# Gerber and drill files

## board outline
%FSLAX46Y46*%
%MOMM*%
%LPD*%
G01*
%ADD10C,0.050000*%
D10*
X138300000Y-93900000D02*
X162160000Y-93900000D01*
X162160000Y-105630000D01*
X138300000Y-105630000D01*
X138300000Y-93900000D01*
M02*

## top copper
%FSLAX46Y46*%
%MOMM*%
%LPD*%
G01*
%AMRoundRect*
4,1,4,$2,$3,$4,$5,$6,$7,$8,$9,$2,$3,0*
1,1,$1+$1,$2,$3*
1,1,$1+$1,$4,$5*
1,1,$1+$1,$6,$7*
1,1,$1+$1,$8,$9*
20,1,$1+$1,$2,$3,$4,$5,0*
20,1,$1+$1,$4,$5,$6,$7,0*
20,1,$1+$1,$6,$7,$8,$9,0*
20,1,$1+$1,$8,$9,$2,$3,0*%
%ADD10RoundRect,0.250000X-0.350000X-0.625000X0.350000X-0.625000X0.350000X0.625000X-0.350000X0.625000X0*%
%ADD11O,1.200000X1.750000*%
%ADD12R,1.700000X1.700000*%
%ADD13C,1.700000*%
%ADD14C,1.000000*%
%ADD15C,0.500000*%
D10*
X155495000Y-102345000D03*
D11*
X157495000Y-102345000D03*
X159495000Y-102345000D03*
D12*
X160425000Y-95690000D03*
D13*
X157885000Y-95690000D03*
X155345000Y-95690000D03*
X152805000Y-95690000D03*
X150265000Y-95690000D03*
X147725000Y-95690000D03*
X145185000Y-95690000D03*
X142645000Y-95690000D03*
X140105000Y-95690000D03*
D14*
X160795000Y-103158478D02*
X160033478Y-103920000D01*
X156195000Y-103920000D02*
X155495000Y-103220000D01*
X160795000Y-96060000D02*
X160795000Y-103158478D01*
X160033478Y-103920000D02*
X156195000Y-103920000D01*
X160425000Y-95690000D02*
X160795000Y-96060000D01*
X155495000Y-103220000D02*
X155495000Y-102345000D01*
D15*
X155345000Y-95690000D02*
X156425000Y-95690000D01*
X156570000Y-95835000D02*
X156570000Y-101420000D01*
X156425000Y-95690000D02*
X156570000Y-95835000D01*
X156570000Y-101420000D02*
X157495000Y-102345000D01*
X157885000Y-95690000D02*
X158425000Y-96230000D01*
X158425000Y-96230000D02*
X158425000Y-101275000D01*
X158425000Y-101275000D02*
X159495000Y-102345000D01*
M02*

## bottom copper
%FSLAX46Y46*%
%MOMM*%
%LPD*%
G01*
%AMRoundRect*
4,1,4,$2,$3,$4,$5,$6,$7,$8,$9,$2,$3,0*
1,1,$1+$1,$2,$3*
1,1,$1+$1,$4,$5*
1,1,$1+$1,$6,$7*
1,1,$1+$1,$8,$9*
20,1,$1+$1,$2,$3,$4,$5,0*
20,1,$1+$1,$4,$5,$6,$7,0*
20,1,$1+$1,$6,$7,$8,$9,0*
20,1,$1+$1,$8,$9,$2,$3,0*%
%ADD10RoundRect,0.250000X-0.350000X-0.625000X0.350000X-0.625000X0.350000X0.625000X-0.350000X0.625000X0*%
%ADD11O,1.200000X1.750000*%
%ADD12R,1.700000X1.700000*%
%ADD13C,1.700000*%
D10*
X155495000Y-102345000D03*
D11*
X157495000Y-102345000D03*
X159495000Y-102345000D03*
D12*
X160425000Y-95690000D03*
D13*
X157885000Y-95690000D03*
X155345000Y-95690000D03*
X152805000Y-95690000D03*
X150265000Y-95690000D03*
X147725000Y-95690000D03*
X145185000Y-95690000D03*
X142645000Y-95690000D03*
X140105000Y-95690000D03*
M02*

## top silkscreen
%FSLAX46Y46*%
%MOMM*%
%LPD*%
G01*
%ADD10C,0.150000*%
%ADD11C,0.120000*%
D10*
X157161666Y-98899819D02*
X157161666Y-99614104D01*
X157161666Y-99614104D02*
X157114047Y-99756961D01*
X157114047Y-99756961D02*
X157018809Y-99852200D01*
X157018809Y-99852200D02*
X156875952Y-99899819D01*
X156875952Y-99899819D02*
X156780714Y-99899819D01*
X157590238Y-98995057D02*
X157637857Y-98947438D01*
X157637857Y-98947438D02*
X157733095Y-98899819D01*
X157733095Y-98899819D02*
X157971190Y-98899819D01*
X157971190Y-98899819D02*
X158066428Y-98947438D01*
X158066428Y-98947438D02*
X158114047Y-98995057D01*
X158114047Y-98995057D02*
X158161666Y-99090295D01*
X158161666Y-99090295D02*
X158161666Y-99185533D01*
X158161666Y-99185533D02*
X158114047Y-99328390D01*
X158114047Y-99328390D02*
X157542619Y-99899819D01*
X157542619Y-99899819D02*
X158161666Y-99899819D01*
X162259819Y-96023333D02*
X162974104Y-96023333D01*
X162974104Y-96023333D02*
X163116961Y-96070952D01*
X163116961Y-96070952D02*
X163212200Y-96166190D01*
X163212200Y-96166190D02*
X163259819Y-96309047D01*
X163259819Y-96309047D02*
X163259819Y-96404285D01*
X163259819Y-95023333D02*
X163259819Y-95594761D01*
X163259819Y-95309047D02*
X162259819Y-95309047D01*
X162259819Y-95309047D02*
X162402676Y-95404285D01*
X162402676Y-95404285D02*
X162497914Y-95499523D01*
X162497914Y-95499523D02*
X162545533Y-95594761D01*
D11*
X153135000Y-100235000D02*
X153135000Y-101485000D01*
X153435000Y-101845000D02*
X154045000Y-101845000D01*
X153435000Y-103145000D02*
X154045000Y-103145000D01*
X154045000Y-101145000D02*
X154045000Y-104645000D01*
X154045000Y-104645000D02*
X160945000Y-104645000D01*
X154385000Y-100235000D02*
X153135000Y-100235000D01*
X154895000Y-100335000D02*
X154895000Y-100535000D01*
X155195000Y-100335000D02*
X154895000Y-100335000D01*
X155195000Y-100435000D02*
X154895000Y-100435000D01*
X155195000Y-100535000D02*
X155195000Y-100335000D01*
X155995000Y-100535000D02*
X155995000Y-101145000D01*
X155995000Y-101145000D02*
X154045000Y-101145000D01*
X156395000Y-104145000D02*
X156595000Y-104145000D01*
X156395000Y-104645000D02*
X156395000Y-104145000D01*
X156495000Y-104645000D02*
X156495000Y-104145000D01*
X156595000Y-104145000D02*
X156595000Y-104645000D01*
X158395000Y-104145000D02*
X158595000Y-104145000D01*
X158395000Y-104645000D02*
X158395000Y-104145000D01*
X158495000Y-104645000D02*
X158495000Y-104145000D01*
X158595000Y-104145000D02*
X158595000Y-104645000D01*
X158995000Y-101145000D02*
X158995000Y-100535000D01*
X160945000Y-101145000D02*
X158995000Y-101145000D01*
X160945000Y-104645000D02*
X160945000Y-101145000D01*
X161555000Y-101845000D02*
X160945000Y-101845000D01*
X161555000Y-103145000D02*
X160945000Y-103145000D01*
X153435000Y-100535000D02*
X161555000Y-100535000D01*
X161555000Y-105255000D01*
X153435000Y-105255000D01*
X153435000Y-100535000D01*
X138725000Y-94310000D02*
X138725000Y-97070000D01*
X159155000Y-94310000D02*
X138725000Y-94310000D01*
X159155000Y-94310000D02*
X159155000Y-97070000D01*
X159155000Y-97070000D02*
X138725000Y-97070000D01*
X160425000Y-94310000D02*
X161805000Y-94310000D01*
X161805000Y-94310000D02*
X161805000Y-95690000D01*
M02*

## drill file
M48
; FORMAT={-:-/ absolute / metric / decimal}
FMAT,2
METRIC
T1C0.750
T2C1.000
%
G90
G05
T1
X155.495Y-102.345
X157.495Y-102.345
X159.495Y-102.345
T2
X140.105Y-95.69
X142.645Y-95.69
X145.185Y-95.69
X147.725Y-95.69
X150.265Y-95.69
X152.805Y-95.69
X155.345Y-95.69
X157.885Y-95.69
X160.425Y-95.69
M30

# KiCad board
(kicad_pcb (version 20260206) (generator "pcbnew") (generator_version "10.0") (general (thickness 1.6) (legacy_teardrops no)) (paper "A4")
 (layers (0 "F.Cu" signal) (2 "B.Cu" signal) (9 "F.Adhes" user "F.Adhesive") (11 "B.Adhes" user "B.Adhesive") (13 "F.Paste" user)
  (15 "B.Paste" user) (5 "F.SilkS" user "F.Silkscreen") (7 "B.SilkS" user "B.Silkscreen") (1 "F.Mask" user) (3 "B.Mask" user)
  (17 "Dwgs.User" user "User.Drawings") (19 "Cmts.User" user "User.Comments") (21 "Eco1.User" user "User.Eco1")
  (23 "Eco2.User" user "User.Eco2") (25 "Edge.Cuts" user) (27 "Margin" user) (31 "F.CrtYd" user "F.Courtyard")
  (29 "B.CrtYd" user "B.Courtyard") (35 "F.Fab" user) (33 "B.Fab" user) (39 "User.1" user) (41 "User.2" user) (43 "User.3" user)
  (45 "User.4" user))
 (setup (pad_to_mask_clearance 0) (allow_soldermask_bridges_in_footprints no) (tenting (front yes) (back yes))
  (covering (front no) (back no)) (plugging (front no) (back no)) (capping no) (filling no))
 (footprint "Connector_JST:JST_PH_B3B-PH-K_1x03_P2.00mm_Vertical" (layer "F.Cu") (at 155.495 102.345)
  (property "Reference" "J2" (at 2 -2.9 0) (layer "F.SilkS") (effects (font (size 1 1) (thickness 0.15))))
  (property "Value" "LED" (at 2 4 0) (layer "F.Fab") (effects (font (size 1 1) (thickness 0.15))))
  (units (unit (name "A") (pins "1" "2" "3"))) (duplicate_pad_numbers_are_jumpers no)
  (fp_line (start -2.36 -2.11) (end -2.36 -0.86) (stroke (width 0.12) (type solid)) (layer "F.SilkS"))
  (fp_line (start -2.06 -0.5) (end -1.45 -0.5) (stroke (width 0.12) (type solid)) (layer "F.SilkS"))
  (fp_line (start -2.06 0.8) (end -1.45 0.8) (stroke (width 0.12) (type solid)) (layer "F.SilkS"))
  (fp_line (start -1.45 -1.2) (end -1.45 2.3) (stroke (width 0.12) (type solid)) (layer "F.SilkS"))
  (fp_line (start -1.45 2.3) (end 5.45 2.3) (stroke (width 0.12) (type solid)) (layer "F.SilkS"))
  (fp_line (start -1.11 -2.11) (end -2.36 -2.11) (stroke (width 0.12) (type solid)) (layer "F.SilkS"))
  (fp_line (start -0.6 -2.01) (end -0.6 -1.81) (stroke (width 0.12) (type solid)) (layer "F.SilkS"))
  (fp_line (start -0.3 -2.01) (end -0.6 -2.01) (stroke (width 0.12) (type solid)) (layer "F.SilkS"))
  (fp_line (start -0.3 -1.91) (end -0.6 -1.91) (stroke (width 0.12) (type solid)) (layer "F.SilkS"))
  (fp_line (start -0.3 -1.81) (end -0.3 -2.01) (stroke (width 0.12) (type solid)) (layer "F.SilkS"))
  (fp_line (start 0.5 -1.81) (end 0.5 -1.2) (stroke (width 0.12) (type solid)) (layer "F.SilkS"))
  (fp_line (start 0.5 -1.2) (end -1.45 -1.2) (stroke (width 0.12) (type solid)) (layer "F.SilkS"))
  (fp_line (start 0.9 1.8) (end 1.1 1.8) (stroke (width 0.12) (type solid)) (layer "F.SilkS"))
  (fp_line (start 0.9 2.3) (end 0.9 1.8) (stroke (width 0.12) (type solid)) (layer "F.SilkS"))
  (fp_line (start 1 2.3) (end 1 1.8) (stroke (width 0.12) (type solid)) (layer "F.SilkS"))
  (fp_line (start 1.1 1.8) (end 1.1 2.3) (stroke (width 0.12) (type solid)) (layer "F.SilkS"))
  (fp_line (start 2.9 1.8) (end 3.1 1.8) (stroke (width 0.12) (type solid)) (layer "F.SilkS"))
  (fp_line (start 2.9 2.3) (end 2.9 1.8) (stroke (width 0.12) (type solid)) (layer "F.SilkS"))
  (fp_line (start 3 2.3) (end 3 1.8) (stroke (width 0.12) (type solid)) (layer "F.SilkS"))
  (fp_line (start 3.1 1.8) (end 3.1 2.3) (stroke (width 0.12) (type solid)) (layer "F.SilkS"))
  (fp_line (start 3.5 -1.2) (end 3.5 -1.81) (stroke (width 0.12) (type solid)) (layer "F.SilkS"))
  (fp_line (start 5.45 -1.2) (end 3.5 -1.2) (stroke (width 0.12) (type solid)) (layer "F.SilkS"))
  (fp_line (start 5.45 2.3) (end 5.45 -1.2) (stroke (width 0.12) (type solid)) (layer "F.SilkS"))
  (fp_line (start 6.06 -0.5) (end 5.45 -0.5) (stroke (width 0.12) (type solid)) (layer "F.SilkS"))
  (fp_line (start 6.06 0.8) (end 5.45 0.8) (stroke (width 0.12) (type solid)) (layer "F.SilkS"))
  (fp_rect (start -2.06 -1.81) (end 6.06 2.91) (stroke (width 0.12) (type solid)) (fill no) (layer "F.SilkS"))
  (pad "1" thru_hole roundrect (at 0 0) (size 1.2 1.75) (drill 0.75) (layers "*.Cu" "*.Mask") (remove_unused_layers no)
   (roundrect_rratio 0.208333) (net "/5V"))
  (pad "2" thru_hole oval (at 2 0) (size 1.2 1.75) (drill 0.75) (layers "*.Cu" "*.Mask") (remove_unused_layers no) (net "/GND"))
  (pad "3" thru_hole oval (at 4 0) (size 1.2 1.75) (drill 0.75) (layers "*.Cu" "*.Mask") (remove_unused_layers no) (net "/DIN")))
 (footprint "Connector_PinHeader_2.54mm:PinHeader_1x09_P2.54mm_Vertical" (layer "F.Cu") (at 160.425 95.69 -90)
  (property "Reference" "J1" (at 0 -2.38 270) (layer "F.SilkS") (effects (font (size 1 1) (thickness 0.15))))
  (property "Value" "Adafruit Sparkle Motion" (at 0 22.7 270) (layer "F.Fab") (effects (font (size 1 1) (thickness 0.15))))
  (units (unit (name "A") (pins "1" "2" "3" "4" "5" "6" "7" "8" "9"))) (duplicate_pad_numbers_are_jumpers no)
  (fp_line (start -1.38 21.7) (end 1.38 21.7) (stroke (width 0.12) (type solid)) (layer "F.SilkS"))
  (fp_line (start -1.38 1.27) (end -1.38 21.7) (stroke (width 0.12) (type solid)) (layer "F.SilkS"))
  (fp_line (start -1.38 1.27) (end 1.38 1.27) (stroke (width 0.12) (type solid)) (layer "F.SilkS"))
  (fp_line (start 1.38 1.27) (end 1.38 21.7) (stroke (width 0.12) (type solid)) (layer "F.SilkS"))
  (fp_line (start -1.38 0) (end -1.38 -1.38) (stroke (width 0.12) (type solid)) (layer "F.SilkS"))
  (fp_line (start -1.38 -1.38) (end 0 -1.38) (stroke (width 0.12) (type solid)) (layer "F.SilkS"))
  (pad "1" thru_hole rect (at 0 0 270) (size 1.7 1.7) (drill 1) (layers "*.Cu" "*.Mask") (remove_unused_layers no) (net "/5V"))
  (pad "2" thru_hole circle (at 0 2.54 270) (size 1.7 1.7) (drill 1) (layers "*.Cu" "*.Mask") (remove_unused_layers no) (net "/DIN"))
  (pad "3" thru_hole circle (at 0 5.08 270) (size 1.7 1.7) (drill 1) (layers "*.Cu" "*.Mask") (remove_unused_layers no) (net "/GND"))
  (pad "4" thru_hole circle (at 0 7.62 270) (size 1.7 1.7) (drill 1) (layers "*.Cu" "*.Mask") (remove_unused_layers no)
   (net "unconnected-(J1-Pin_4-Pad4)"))
  (pad "5" thru_hole circle (at 0 10.16 270) (size 1.7 1.7) (drill 1) (layers "*.Cu" "*.Mask") (remove_unused_layers no)
   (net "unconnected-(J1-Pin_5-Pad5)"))
  (pad "6" thru_hole circle (at 0 12.7 270) (size 1.7 1.7) (drill 1) (layers "*.Cu" "*.Mask") (remove_unused_layers no)
   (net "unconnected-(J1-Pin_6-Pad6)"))
  (pad "7" thru_hole circle (at 0 15.24 270) (size 1.7 1.7) (drill 1) (layers "*.Cu" "*.Mask") (remove_unused_layers no)
   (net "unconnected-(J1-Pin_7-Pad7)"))
  (pad "8" thru_hole circle (at 0 17.78 270) (size 1.7 1.7) (drill 1) (layers "*.Cu" "*.Mask") (remove_unused_layers no)
   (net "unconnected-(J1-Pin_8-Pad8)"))
  (pad "9" thru_hole circle (at 0 20.32 270) (size 1.7 1.7) (drill 1) (layers "*.Cu" "*.Mask") (remove_unused_layers no)
   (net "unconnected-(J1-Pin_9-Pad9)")))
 (gr_rect (start 138.3 93.9) (end 162.16 105.63) (stroke (width 0.05) (type default)) (fill no) (layer "Edge.Cuts"))
 (segment (start 160.795 103.158478) (end 160.033478 103.92) (width 1) (layer "F.Cu") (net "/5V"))
 (segment (start 156.195 103.92) (end 155.495 103.22) (width 1) (layer "F.Cu") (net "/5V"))
 (segment (start 160.795 96.06) (end 160.795 103.158478) (width 1) (layer "F.Cu") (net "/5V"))
 (segment (start 160.033478 103.92) (end 156.195 103.92) (width 1) (layer "F.Cu") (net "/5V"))
 (segment (start 160.425 95.69) (end 160.795 96.06) (width 1) (layer "F.Cu") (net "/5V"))
 (segment (start 155.495 103.22) (end 155.495 102.345) (width 1) (layer "F.Cu") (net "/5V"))
 (segment (start 155.345 95.69) (end 156.425 95.69) (width 0.5) (layer "F.Cu") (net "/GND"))
 (segment (start 156.57 95.835) (end 156.57 101.42) (width 0.5) (layer "F.Cu") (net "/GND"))
 (segment (start 156.425 95.69) (end 156.57 95.835) (width 0.5) (layer "F.Cu") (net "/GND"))
 (segment (start 156.57 101.42) (end 157.495 102.345) (width 0.5) (layer "F.Cu") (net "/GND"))
 (segment (start 157.885 95.69) (end 158.425 96.23) (width 0.5) (layer "F.Cu") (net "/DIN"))
 (segment (start 158.425 96.23) (end 158.425 101.275) (width 0.5) (layer "F.Cu") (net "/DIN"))
 (segment (start 158.425 101.275) (end 159.495 102.345) (width 0.5) (layer "F.Cu") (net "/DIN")))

